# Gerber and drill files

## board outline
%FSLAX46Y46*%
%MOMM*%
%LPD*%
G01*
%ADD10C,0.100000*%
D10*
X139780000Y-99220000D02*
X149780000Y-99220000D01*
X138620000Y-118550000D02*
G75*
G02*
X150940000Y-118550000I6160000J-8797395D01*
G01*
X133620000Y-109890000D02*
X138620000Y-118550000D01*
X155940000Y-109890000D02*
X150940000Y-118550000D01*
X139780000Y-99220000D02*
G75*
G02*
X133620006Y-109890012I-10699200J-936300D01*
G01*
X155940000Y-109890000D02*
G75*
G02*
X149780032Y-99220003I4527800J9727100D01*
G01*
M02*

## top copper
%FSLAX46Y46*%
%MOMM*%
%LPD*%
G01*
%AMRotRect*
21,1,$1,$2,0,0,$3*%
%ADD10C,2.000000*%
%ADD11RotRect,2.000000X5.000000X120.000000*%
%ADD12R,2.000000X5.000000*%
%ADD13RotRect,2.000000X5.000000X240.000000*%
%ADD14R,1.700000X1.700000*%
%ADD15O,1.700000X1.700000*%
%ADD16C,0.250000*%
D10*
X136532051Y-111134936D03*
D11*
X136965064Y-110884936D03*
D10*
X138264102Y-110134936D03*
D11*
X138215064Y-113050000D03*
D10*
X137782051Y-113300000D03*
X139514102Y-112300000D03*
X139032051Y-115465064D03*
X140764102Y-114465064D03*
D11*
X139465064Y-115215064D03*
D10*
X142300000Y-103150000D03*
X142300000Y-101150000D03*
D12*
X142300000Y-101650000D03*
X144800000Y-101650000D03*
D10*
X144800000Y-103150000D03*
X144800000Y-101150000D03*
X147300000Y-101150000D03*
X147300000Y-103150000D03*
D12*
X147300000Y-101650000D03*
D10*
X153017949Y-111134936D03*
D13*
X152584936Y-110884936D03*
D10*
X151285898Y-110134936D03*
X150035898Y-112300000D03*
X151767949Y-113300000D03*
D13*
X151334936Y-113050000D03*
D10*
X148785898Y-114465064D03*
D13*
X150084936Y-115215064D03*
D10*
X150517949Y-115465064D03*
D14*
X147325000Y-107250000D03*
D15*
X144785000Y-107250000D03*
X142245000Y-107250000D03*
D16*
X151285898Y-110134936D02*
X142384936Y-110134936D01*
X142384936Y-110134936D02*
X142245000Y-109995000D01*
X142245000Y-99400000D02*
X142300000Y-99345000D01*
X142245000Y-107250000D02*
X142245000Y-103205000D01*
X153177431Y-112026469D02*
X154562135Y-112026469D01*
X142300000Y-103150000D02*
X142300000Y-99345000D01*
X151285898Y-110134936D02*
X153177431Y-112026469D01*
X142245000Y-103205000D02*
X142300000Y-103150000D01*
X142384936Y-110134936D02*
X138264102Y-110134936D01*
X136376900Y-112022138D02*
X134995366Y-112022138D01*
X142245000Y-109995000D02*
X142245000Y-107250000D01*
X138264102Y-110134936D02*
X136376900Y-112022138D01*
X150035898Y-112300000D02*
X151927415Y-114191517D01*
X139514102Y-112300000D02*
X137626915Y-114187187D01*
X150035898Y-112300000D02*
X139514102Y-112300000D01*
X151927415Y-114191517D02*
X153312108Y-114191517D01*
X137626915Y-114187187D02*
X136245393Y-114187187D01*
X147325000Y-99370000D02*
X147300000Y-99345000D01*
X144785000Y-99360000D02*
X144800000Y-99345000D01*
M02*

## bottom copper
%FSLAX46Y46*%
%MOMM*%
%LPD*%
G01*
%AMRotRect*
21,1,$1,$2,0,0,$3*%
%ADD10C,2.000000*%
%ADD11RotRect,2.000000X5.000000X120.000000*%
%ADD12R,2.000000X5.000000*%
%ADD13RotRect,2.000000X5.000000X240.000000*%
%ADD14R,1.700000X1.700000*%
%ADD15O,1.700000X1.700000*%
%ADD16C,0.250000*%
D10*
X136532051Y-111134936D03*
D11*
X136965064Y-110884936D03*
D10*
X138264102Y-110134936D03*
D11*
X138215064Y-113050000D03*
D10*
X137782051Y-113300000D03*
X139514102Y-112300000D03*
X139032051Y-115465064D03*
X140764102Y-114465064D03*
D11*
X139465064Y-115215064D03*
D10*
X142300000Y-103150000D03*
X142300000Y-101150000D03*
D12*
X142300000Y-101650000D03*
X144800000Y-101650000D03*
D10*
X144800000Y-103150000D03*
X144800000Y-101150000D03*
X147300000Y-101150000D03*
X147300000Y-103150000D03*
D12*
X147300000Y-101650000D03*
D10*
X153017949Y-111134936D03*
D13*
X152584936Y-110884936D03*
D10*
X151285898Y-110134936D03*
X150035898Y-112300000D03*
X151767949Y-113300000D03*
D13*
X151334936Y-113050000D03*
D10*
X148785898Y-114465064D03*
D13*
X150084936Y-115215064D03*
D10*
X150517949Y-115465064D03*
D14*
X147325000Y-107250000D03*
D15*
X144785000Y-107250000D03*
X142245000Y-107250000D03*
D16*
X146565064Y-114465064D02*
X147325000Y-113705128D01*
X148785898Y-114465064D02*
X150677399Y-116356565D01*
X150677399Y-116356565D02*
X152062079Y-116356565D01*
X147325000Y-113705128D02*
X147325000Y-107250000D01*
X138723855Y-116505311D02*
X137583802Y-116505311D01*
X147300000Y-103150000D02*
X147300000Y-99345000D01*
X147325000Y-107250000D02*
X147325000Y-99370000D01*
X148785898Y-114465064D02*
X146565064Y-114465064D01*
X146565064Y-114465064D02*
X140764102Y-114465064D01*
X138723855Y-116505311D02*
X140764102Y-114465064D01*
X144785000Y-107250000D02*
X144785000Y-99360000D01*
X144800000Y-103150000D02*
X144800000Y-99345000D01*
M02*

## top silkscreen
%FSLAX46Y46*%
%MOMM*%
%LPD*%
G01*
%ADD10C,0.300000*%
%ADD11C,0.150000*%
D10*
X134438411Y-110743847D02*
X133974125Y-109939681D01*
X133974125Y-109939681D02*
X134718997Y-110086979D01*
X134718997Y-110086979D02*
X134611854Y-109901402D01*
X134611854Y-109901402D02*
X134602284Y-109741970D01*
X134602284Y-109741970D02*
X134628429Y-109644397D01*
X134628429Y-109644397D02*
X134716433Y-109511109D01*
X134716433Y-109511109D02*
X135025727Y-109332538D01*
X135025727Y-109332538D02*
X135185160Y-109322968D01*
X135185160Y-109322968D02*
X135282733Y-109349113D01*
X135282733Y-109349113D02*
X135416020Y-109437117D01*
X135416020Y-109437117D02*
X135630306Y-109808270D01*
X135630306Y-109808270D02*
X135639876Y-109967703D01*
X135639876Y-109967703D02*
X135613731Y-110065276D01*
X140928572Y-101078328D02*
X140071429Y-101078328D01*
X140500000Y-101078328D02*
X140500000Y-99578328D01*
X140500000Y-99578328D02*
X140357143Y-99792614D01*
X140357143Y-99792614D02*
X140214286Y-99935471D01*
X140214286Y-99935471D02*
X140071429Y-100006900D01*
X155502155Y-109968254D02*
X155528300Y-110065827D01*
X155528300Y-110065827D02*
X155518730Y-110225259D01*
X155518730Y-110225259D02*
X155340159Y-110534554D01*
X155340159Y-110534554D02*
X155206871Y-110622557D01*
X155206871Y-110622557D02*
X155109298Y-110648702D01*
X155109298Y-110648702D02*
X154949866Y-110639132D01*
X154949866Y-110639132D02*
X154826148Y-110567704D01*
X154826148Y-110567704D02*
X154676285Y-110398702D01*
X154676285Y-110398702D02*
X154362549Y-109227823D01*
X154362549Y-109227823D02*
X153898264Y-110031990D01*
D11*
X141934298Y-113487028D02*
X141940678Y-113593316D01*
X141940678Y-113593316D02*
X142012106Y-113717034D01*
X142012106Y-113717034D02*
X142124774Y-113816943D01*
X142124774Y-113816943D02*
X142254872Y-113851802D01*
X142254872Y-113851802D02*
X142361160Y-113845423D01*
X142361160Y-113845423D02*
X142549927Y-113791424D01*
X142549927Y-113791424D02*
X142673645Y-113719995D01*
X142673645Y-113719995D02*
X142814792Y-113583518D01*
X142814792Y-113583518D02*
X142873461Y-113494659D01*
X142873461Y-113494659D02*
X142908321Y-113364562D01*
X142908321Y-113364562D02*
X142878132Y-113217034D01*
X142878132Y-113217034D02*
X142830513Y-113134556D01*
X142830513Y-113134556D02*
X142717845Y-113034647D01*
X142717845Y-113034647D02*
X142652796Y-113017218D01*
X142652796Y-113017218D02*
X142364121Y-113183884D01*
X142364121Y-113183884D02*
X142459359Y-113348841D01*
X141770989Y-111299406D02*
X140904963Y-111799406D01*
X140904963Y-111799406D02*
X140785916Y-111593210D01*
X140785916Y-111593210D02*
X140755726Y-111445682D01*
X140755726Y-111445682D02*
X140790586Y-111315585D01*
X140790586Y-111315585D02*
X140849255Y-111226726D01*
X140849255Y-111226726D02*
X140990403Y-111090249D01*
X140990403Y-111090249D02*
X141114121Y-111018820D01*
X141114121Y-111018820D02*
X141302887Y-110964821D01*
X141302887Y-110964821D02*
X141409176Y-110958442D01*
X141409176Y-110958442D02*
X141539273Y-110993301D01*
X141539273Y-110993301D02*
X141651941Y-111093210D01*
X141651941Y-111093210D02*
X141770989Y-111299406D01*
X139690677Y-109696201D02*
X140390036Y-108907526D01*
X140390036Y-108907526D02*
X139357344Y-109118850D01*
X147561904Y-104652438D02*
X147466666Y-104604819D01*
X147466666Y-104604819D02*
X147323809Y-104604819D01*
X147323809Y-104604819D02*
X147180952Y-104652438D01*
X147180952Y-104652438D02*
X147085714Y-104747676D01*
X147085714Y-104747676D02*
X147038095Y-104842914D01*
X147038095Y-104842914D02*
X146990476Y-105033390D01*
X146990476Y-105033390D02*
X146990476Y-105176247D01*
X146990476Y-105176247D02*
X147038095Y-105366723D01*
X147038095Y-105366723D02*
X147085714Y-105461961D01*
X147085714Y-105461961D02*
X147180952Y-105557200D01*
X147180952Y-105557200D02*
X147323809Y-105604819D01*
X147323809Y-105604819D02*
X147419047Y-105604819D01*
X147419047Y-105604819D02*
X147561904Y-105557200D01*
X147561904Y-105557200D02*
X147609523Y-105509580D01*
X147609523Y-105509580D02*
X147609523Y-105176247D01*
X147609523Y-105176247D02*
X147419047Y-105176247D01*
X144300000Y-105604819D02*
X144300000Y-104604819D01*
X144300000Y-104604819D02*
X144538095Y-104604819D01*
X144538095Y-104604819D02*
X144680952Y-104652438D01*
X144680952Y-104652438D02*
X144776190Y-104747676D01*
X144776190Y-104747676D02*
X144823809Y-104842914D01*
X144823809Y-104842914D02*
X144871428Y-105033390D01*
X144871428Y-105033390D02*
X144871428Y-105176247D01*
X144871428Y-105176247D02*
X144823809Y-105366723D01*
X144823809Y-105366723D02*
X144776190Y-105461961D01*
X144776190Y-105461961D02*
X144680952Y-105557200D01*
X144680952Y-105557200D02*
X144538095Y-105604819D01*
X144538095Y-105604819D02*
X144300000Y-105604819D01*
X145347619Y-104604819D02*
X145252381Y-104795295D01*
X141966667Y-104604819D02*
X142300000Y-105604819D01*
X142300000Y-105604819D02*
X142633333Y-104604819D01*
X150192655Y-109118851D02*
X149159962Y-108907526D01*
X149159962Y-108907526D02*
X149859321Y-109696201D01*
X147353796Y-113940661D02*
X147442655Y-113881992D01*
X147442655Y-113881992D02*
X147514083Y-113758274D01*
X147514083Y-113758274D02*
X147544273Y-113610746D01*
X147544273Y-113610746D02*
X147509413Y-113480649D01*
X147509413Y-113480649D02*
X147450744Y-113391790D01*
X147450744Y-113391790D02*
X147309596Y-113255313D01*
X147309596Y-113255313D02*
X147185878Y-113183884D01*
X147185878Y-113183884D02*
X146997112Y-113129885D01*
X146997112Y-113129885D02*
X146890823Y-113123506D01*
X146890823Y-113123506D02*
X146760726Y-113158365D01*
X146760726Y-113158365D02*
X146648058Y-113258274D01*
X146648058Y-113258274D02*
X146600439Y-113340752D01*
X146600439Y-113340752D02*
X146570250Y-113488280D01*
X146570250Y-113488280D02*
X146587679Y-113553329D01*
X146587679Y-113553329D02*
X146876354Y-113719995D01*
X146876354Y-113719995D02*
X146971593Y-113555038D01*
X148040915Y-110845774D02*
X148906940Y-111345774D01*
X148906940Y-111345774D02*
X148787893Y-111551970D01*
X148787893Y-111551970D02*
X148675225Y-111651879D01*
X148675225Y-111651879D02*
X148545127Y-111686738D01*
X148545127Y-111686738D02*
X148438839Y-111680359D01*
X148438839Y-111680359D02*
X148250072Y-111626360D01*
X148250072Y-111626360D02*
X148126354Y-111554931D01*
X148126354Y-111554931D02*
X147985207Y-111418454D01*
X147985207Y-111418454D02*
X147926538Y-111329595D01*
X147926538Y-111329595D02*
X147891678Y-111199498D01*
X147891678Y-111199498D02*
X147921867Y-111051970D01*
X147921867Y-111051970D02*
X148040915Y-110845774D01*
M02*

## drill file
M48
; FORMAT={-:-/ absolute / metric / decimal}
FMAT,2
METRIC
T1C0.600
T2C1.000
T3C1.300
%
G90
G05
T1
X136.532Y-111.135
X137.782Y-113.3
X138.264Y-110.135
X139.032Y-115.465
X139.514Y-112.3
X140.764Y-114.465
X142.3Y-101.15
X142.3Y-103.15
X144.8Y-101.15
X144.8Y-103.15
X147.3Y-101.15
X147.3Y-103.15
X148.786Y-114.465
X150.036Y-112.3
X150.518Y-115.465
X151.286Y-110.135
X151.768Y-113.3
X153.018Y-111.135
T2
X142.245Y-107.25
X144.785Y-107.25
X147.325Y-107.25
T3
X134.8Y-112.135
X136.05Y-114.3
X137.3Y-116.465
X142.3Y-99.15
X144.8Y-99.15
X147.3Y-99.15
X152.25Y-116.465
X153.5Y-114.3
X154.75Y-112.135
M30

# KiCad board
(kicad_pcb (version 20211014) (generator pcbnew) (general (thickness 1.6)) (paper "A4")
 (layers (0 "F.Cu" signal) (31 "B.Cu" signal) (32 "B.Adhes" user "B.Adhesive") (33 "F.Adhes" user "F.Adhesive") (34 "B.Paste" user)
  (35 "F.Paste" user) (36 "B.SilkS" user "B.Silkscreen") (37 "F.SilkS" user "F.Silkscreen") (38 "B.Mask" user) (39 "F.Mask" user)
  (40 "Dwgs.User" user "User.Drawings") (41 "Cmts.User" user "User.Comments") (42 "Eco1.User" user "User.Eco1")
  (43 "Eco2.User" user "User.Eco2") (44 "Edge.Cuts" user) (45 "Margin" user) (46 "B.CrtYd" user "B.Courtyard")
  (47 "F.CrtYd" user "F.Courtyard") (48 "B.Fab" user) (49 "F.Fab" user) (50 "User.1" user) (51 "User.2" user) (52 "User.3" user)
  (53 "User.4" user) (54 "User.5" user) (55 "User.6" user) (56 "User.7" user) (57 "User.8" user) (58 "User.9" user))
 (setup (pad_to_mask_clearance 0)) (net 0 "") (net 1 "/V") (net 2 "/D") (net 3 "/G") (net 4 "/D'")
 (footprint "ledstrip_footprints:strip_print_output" (layer "F.Cu") (at 136.05 114.3 120)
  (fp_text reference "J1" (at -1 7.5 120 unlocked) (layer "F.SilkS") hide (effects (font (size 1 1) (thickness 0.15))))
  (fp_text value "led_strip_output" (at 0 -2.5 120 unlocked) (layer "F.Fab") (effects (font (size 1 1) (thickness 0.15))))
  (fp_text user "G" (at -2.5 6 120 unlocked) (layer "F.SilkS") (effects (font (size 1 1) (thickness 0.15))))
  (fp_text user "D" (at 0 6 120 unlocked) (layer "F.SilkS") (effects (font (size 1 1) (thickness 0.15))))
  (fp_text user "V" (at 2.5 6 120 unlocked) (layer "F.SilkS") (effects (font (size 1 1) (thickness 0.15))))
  (pad "1" thru_hole circle (at 2.5 2 120) (size 2 2) (drill 0.6) (layers *.Cu *.Mask) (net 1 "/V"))
  (pad "1" thru_hole rect (at 2.5 0 120) (size 2 5) (drill 1.3 (offset 0 2.5)) (layers *.Cu *.Mask) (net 1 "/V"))
  (pad "1" thru_hole circle (at 2.5 4 120) (size 2 2) (drill 0.6) (layers *.Cu *.Mask) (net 1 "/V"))
  (pad "2" thru_hole rect (at 0 0 120) (size 2 5) (drill 1.3 (offset 0 2.5)) (layers *.Cu *.Mask) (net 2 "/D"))
  (pad "2" thru_hole circle (at 0 2 120) (size 2 2) (drill 0.6) (layers *.Cu *.Mask) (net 2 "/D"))
  (pad "2" thru_hole circle (at 0 4 120) (size 2 2) (drill 0.6) (layers *.Cu *.Mask) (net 2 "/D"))
  (pad "3" thru_hole circle (at -2.5 2 120) (size 2 2) (drill 0.6) (layers *.Cu *.Mask) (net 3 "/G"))
  (pad "3" thru_hole circle (at -2.5 4 120) (size 2 2) (drill 0.6) (layers *.Cu *.Mask) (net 3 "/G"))
  (pad "3" thru_hole rect (at -2.5 0 120) (size 2 5) (drill 1.3 (offset 0 2.5)) (layers *.Cu *.Mask) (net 3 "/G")))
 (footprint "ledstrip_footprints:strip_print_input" (layer "F.Cu") (at 144.8 99.15)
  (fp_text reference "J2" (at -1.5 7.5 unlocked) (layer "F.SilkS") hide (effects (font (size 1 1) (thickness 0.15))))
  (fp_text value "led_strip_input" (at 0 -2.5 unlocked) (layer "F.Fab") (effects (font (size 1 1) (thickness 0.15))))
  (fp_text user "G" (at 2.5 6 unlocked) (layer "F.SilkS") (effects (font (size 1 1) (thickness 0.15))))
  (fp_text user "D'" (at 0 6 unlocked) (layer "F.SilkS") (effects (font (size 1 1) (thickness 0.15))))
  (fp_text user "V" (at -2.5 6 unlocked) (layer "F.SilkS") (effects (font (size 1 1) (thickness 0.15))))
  (pad "1" thru_hole circle (at -2.5 4) (size 2 2) (drill 0.6) (layers *.Cu *.Mask) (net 1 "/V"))
  (pad "1" thru_hole circle (at -2.5 2) (size 2 2) (drill 0.6) (layers *.Cu *.Mask) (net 1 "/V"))
  (pad "1" thru_hole rect (at -2.5 0) (size 2 5) (drill 1.3 (offset 0 2.5)) (layers *.Cu *.Mask) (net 1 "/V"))
  (pad "2" thru_hole rect (at 0 0) (size 2 5) (drill 1.3 (offset 0 2.5)) (layers *.Cu *.Mask) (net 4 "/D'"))
  (pad "2" thru_hole circle (at 0 4) (size 2 2) (drill 0.6) (layers *.Cu *.Mask) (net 4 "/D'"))
  (pad "2" thru_hole circle (at 0 2) (size 2 2) (drill 0.6) (layers *.Cu *.Mask) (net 4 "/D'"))
  (pad "3" thru_hole circle (at 2.5 2) (size 2 2) (drill 0.6) (layers *.Cu *.Mask) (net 3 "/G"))
  (pad "3" thru_hole circle (at 2.5 4) (size 2 2) (drill 0.6) (layers *.Cu *.Mask) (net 3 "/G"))
  (pad "3" thru_hole rect (at 2.5 0) (size 2 5) (drill 1.3 (offset 0 2.5)) (layers *.Cu *.Mask) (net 3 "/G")))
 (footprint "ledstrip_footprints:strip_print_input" (layer "F.Cu") (at 153.5 114.3 -120)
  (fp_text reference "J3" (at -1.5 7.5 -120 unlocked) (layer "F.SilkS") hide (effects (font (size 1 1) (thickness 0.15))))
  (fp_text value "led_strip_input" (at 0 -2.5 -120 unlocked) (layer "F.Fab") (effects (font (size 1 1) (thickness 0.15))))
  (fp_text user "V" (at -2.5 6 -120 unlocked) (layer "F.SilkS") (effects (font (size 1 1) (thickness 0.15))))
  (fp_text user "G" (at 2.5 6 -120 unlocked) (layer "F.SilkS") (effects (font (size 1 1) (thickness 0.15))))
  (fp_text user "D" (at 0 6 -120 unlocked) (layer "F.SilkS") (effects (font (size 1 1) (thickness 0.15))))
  (pad "1" thru_hole circle (at -2.5 2 240) (size 2 2) (drill 0.6) (layers *.Cu *.Mask) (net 1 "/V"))
  (pad "1" thru_hole rect (at -2.5 0 240) (size 2 5) (drill 1.3 (offset 0 2.5)) (layers *.Cu *.Mask) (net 1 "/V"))
  (pad "1" thru_hole circle (at -2.5 4 240) (size 2 2) (drill 0.6) (layers *.Cu *.Mask) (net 1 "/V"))
  (pad "2" thru_hole circle (at 0 4 240) (size 2 2) (drill 0.6) (layers *.Cu *.Mask) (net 2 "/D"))
  (pad "2" thru_hole circle (at 0 2 240) (size 2 2) (drill 0.6) (layers *.Cu *.Mask) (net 2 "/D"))
  (pad "2" thru_hole rect (at 0 0 240) (size 2 5) (drill 1.3 (offset 0 2.5)) (layers *.Cu *.Mask) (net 2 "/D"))
  (pad "3" thru_hole circle (at 2.5 4 240) (size 2 2) (drill 0.6) (layers *.Cu *.Mask) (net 3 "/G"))
  (pad "3" thru_hole rect (at 2.5 0 240) (size 2 5) (drill 1.3 (offset 0 2.5)) (layers *.Cu *.Mask) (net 3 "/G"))
  (pad "3" thru_hole circle (at 2.5 2 240) (size 2 2) (drill 0.6) (layers *.Cu *.Mask) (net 3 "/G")))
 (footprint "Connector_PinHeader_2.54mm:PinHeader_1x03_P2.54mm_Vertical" (layer "B.Cu") (at 147.325 107.25 90)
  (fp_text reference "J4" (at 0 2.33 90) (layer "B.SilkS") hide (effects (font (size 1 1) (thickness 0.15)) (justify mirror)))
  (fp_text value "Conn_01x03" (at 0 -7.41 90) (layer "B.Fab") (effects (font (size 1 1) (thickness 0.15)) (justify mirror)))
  (pad "1" thru_hole rect (at 0 0 90) (size 1.7 1.7) (drill 1) (layers *.Cu *.Mask) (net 3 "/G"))
  (pad "2" thru_hole oval (at 0 -2.54 90) (size 1.7 1.7) (drill 1) (layers *.Cu *.Mask) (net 4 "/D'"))
  (pad "3" thru_hole oval (at 0 -5.08 90) (size 1.7 1.7) (drill 1) (layers *.Cu *.Mask) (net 1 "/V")))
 (gr_line (start 139.78 99.22) (end 149.78 99.22) (layer "Edge.Cuts") (width 0.1))
 (gr_arc (start 138.62 118.55) (mid 144.78 116.60776) (end 150.94 118.55) (layer "Edge.Cuts") (width 0.1))
 (gr_line (start 133.62 109.89) (end 138.62 118.55) (layer "Edge.Cuts") (width 0.1))
 (gr_line (start 155.94 109.89) (end 150.94 118.55) (layer "Edge.Cuts") (width 0.1))
 (gr_arc (start 139.78 99.22) (mid 138.382119 105.52612) (end 133.62 109.89) (layer "Edge.Cuts") (width 0.1))
 (gr_arc (start 155.94 109.89) (mid 151.17582 105.52731) (end 149.78 99.22) (layer "Edge.Cuts") (width 0.1))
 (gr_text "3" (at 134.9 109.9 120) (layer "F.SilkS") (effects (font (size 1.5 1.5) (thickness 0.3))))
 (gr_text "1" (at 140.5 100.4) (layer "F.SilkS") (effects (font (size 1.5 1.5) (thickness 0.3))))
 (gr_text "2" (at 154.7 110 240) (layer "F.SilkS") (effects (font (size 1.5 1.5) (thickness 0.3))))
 (segment (start 151.285898 110.134936) (end 142.384936 110.134936) (width 0.25) (layer "F.Cu") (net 1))
 (segment (start 142.384936 110.134936) (end 142.245 109.995) (width 0.25) (layer "F.Cu") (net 1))
 (segment (start 142.245 99.4) (end 142.3 99.345) (width 0.25) (layer "F.Cu") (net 1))
 (segment (start 142.245 107.25) (end 142.245 103.205) (width 0.25) (layer "F.Cu") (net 1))
 (segment (start 153.177431 112.026469) (end 154.562135 112.026469) (width 0.25) (layer "F.Cu") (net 1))
 (segment (start 142.3 103.15) (end 142.3 99.345) (width 0.25) (layer "F.Cu") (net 1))
 (segment (start 151.285898 110.134936) (end 153.177431 112.026469) (width 0.25) (layer "F.Cu") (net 1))
 (segment (start 142.245 103.205) (end 142.3 103.15) (width 0.25) (layer "F.Cu") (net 1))
 (segment (start 142.384936 110.134936) (end 138.264102 110.134936) (width 0.25) (layer "F.Cu") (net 1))
 (segment (start 136.3769 112.022138) (end 134.995366 112.022138) (width 0.25) (layer "F.Cu") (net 1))
 (segment (start 142.245 109.995) (end 142.245 107.25) (width 0.25) (layer "F.Cu") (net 1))
 (segment (start 138.264102 110.134936) (end 136.3769 112.022138) (width 0.25) (layer "F.Cu") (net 1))
 (segment (start 150.035898 112.3) (end 151.927415 114.191517) (width 0.25) (layer "F.Cu") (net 2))
 (segment (start 139.514102 112.3) (end 137.626915 114.187187) (width 0.25) (layer "F.Cu") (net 2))
 (segment (start 150.035898 112.3) (end 139.514102 112.3) (width 0.25) (layer "F.Cu") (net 2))
 (segment (start 151.927415 114.191517) (end 153.312108 114.191517) (width 0.25) (layer "F.Cu") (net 2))
 (segment (start 137.626915 114.187187) (end 136.245393 114.187187) (width 0.25) (layer "F.Cu") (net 2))
 (segment (start 147.325 99.37) (end 147.3 99.345) (width 0.25) (layer "F.Cu") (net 3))
 (segment (start 146.565064 114.465064) (end 147.325 113.705128) (width 0.25) (layer "B.Cu") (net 3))
 (segment (start 148.785898 114.465064) (end 150.677399 116.356565) (width 0.25) (layer "B.Cu") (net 3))
 (segment (start 150.677399 116.356565) (end 152.062079 116.356565) (width 0.25) (layer "B.Cu") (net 3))
 (segment (start 147.325 113.705128) (end 147.325 107.25) (width 0.25) (layer "B.Cu") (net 3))
 (segment (start 138.723855 116.505311) (end 137.583802 116.505311) (width 0.25) (layer "B.Cu") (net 3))
 (segment (start 147.3 103.15) (end 147.3 99.345) (width 0.25) (layer "B.Cu") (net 3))
 (segment (start 147.325 107.25) (end 147.325 99.37) (width 0.25) (layer "B.Cu") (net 3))
 (segment (start 148.785898 114.465064) (end 146.565064 114.465064) (width 0.25) (layer "B.Cu") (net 3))
 (segment (start 146.565064 114.465064) (end 140.764102 114.465064) (width 0.25) (layer "B.Cu") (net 3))
 (segment (start 138.723855 116.505311) (end 140.764102 114.465064) (width 0.25) (layer "B.Cu") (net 3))
 (segment (start 144.785 99.36) (end 144.8 99.345) (width 0.25) (layer "F.Cu") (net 4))
 (segment (start 144.785 107.25) (end 144.785 99.36) (width 0.25) (layer "B.Cu") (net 4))
 (segment (start 144.8 103.15) (end 144.8 99.345) (width 0.25) (layer "B.Cu") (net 4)))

